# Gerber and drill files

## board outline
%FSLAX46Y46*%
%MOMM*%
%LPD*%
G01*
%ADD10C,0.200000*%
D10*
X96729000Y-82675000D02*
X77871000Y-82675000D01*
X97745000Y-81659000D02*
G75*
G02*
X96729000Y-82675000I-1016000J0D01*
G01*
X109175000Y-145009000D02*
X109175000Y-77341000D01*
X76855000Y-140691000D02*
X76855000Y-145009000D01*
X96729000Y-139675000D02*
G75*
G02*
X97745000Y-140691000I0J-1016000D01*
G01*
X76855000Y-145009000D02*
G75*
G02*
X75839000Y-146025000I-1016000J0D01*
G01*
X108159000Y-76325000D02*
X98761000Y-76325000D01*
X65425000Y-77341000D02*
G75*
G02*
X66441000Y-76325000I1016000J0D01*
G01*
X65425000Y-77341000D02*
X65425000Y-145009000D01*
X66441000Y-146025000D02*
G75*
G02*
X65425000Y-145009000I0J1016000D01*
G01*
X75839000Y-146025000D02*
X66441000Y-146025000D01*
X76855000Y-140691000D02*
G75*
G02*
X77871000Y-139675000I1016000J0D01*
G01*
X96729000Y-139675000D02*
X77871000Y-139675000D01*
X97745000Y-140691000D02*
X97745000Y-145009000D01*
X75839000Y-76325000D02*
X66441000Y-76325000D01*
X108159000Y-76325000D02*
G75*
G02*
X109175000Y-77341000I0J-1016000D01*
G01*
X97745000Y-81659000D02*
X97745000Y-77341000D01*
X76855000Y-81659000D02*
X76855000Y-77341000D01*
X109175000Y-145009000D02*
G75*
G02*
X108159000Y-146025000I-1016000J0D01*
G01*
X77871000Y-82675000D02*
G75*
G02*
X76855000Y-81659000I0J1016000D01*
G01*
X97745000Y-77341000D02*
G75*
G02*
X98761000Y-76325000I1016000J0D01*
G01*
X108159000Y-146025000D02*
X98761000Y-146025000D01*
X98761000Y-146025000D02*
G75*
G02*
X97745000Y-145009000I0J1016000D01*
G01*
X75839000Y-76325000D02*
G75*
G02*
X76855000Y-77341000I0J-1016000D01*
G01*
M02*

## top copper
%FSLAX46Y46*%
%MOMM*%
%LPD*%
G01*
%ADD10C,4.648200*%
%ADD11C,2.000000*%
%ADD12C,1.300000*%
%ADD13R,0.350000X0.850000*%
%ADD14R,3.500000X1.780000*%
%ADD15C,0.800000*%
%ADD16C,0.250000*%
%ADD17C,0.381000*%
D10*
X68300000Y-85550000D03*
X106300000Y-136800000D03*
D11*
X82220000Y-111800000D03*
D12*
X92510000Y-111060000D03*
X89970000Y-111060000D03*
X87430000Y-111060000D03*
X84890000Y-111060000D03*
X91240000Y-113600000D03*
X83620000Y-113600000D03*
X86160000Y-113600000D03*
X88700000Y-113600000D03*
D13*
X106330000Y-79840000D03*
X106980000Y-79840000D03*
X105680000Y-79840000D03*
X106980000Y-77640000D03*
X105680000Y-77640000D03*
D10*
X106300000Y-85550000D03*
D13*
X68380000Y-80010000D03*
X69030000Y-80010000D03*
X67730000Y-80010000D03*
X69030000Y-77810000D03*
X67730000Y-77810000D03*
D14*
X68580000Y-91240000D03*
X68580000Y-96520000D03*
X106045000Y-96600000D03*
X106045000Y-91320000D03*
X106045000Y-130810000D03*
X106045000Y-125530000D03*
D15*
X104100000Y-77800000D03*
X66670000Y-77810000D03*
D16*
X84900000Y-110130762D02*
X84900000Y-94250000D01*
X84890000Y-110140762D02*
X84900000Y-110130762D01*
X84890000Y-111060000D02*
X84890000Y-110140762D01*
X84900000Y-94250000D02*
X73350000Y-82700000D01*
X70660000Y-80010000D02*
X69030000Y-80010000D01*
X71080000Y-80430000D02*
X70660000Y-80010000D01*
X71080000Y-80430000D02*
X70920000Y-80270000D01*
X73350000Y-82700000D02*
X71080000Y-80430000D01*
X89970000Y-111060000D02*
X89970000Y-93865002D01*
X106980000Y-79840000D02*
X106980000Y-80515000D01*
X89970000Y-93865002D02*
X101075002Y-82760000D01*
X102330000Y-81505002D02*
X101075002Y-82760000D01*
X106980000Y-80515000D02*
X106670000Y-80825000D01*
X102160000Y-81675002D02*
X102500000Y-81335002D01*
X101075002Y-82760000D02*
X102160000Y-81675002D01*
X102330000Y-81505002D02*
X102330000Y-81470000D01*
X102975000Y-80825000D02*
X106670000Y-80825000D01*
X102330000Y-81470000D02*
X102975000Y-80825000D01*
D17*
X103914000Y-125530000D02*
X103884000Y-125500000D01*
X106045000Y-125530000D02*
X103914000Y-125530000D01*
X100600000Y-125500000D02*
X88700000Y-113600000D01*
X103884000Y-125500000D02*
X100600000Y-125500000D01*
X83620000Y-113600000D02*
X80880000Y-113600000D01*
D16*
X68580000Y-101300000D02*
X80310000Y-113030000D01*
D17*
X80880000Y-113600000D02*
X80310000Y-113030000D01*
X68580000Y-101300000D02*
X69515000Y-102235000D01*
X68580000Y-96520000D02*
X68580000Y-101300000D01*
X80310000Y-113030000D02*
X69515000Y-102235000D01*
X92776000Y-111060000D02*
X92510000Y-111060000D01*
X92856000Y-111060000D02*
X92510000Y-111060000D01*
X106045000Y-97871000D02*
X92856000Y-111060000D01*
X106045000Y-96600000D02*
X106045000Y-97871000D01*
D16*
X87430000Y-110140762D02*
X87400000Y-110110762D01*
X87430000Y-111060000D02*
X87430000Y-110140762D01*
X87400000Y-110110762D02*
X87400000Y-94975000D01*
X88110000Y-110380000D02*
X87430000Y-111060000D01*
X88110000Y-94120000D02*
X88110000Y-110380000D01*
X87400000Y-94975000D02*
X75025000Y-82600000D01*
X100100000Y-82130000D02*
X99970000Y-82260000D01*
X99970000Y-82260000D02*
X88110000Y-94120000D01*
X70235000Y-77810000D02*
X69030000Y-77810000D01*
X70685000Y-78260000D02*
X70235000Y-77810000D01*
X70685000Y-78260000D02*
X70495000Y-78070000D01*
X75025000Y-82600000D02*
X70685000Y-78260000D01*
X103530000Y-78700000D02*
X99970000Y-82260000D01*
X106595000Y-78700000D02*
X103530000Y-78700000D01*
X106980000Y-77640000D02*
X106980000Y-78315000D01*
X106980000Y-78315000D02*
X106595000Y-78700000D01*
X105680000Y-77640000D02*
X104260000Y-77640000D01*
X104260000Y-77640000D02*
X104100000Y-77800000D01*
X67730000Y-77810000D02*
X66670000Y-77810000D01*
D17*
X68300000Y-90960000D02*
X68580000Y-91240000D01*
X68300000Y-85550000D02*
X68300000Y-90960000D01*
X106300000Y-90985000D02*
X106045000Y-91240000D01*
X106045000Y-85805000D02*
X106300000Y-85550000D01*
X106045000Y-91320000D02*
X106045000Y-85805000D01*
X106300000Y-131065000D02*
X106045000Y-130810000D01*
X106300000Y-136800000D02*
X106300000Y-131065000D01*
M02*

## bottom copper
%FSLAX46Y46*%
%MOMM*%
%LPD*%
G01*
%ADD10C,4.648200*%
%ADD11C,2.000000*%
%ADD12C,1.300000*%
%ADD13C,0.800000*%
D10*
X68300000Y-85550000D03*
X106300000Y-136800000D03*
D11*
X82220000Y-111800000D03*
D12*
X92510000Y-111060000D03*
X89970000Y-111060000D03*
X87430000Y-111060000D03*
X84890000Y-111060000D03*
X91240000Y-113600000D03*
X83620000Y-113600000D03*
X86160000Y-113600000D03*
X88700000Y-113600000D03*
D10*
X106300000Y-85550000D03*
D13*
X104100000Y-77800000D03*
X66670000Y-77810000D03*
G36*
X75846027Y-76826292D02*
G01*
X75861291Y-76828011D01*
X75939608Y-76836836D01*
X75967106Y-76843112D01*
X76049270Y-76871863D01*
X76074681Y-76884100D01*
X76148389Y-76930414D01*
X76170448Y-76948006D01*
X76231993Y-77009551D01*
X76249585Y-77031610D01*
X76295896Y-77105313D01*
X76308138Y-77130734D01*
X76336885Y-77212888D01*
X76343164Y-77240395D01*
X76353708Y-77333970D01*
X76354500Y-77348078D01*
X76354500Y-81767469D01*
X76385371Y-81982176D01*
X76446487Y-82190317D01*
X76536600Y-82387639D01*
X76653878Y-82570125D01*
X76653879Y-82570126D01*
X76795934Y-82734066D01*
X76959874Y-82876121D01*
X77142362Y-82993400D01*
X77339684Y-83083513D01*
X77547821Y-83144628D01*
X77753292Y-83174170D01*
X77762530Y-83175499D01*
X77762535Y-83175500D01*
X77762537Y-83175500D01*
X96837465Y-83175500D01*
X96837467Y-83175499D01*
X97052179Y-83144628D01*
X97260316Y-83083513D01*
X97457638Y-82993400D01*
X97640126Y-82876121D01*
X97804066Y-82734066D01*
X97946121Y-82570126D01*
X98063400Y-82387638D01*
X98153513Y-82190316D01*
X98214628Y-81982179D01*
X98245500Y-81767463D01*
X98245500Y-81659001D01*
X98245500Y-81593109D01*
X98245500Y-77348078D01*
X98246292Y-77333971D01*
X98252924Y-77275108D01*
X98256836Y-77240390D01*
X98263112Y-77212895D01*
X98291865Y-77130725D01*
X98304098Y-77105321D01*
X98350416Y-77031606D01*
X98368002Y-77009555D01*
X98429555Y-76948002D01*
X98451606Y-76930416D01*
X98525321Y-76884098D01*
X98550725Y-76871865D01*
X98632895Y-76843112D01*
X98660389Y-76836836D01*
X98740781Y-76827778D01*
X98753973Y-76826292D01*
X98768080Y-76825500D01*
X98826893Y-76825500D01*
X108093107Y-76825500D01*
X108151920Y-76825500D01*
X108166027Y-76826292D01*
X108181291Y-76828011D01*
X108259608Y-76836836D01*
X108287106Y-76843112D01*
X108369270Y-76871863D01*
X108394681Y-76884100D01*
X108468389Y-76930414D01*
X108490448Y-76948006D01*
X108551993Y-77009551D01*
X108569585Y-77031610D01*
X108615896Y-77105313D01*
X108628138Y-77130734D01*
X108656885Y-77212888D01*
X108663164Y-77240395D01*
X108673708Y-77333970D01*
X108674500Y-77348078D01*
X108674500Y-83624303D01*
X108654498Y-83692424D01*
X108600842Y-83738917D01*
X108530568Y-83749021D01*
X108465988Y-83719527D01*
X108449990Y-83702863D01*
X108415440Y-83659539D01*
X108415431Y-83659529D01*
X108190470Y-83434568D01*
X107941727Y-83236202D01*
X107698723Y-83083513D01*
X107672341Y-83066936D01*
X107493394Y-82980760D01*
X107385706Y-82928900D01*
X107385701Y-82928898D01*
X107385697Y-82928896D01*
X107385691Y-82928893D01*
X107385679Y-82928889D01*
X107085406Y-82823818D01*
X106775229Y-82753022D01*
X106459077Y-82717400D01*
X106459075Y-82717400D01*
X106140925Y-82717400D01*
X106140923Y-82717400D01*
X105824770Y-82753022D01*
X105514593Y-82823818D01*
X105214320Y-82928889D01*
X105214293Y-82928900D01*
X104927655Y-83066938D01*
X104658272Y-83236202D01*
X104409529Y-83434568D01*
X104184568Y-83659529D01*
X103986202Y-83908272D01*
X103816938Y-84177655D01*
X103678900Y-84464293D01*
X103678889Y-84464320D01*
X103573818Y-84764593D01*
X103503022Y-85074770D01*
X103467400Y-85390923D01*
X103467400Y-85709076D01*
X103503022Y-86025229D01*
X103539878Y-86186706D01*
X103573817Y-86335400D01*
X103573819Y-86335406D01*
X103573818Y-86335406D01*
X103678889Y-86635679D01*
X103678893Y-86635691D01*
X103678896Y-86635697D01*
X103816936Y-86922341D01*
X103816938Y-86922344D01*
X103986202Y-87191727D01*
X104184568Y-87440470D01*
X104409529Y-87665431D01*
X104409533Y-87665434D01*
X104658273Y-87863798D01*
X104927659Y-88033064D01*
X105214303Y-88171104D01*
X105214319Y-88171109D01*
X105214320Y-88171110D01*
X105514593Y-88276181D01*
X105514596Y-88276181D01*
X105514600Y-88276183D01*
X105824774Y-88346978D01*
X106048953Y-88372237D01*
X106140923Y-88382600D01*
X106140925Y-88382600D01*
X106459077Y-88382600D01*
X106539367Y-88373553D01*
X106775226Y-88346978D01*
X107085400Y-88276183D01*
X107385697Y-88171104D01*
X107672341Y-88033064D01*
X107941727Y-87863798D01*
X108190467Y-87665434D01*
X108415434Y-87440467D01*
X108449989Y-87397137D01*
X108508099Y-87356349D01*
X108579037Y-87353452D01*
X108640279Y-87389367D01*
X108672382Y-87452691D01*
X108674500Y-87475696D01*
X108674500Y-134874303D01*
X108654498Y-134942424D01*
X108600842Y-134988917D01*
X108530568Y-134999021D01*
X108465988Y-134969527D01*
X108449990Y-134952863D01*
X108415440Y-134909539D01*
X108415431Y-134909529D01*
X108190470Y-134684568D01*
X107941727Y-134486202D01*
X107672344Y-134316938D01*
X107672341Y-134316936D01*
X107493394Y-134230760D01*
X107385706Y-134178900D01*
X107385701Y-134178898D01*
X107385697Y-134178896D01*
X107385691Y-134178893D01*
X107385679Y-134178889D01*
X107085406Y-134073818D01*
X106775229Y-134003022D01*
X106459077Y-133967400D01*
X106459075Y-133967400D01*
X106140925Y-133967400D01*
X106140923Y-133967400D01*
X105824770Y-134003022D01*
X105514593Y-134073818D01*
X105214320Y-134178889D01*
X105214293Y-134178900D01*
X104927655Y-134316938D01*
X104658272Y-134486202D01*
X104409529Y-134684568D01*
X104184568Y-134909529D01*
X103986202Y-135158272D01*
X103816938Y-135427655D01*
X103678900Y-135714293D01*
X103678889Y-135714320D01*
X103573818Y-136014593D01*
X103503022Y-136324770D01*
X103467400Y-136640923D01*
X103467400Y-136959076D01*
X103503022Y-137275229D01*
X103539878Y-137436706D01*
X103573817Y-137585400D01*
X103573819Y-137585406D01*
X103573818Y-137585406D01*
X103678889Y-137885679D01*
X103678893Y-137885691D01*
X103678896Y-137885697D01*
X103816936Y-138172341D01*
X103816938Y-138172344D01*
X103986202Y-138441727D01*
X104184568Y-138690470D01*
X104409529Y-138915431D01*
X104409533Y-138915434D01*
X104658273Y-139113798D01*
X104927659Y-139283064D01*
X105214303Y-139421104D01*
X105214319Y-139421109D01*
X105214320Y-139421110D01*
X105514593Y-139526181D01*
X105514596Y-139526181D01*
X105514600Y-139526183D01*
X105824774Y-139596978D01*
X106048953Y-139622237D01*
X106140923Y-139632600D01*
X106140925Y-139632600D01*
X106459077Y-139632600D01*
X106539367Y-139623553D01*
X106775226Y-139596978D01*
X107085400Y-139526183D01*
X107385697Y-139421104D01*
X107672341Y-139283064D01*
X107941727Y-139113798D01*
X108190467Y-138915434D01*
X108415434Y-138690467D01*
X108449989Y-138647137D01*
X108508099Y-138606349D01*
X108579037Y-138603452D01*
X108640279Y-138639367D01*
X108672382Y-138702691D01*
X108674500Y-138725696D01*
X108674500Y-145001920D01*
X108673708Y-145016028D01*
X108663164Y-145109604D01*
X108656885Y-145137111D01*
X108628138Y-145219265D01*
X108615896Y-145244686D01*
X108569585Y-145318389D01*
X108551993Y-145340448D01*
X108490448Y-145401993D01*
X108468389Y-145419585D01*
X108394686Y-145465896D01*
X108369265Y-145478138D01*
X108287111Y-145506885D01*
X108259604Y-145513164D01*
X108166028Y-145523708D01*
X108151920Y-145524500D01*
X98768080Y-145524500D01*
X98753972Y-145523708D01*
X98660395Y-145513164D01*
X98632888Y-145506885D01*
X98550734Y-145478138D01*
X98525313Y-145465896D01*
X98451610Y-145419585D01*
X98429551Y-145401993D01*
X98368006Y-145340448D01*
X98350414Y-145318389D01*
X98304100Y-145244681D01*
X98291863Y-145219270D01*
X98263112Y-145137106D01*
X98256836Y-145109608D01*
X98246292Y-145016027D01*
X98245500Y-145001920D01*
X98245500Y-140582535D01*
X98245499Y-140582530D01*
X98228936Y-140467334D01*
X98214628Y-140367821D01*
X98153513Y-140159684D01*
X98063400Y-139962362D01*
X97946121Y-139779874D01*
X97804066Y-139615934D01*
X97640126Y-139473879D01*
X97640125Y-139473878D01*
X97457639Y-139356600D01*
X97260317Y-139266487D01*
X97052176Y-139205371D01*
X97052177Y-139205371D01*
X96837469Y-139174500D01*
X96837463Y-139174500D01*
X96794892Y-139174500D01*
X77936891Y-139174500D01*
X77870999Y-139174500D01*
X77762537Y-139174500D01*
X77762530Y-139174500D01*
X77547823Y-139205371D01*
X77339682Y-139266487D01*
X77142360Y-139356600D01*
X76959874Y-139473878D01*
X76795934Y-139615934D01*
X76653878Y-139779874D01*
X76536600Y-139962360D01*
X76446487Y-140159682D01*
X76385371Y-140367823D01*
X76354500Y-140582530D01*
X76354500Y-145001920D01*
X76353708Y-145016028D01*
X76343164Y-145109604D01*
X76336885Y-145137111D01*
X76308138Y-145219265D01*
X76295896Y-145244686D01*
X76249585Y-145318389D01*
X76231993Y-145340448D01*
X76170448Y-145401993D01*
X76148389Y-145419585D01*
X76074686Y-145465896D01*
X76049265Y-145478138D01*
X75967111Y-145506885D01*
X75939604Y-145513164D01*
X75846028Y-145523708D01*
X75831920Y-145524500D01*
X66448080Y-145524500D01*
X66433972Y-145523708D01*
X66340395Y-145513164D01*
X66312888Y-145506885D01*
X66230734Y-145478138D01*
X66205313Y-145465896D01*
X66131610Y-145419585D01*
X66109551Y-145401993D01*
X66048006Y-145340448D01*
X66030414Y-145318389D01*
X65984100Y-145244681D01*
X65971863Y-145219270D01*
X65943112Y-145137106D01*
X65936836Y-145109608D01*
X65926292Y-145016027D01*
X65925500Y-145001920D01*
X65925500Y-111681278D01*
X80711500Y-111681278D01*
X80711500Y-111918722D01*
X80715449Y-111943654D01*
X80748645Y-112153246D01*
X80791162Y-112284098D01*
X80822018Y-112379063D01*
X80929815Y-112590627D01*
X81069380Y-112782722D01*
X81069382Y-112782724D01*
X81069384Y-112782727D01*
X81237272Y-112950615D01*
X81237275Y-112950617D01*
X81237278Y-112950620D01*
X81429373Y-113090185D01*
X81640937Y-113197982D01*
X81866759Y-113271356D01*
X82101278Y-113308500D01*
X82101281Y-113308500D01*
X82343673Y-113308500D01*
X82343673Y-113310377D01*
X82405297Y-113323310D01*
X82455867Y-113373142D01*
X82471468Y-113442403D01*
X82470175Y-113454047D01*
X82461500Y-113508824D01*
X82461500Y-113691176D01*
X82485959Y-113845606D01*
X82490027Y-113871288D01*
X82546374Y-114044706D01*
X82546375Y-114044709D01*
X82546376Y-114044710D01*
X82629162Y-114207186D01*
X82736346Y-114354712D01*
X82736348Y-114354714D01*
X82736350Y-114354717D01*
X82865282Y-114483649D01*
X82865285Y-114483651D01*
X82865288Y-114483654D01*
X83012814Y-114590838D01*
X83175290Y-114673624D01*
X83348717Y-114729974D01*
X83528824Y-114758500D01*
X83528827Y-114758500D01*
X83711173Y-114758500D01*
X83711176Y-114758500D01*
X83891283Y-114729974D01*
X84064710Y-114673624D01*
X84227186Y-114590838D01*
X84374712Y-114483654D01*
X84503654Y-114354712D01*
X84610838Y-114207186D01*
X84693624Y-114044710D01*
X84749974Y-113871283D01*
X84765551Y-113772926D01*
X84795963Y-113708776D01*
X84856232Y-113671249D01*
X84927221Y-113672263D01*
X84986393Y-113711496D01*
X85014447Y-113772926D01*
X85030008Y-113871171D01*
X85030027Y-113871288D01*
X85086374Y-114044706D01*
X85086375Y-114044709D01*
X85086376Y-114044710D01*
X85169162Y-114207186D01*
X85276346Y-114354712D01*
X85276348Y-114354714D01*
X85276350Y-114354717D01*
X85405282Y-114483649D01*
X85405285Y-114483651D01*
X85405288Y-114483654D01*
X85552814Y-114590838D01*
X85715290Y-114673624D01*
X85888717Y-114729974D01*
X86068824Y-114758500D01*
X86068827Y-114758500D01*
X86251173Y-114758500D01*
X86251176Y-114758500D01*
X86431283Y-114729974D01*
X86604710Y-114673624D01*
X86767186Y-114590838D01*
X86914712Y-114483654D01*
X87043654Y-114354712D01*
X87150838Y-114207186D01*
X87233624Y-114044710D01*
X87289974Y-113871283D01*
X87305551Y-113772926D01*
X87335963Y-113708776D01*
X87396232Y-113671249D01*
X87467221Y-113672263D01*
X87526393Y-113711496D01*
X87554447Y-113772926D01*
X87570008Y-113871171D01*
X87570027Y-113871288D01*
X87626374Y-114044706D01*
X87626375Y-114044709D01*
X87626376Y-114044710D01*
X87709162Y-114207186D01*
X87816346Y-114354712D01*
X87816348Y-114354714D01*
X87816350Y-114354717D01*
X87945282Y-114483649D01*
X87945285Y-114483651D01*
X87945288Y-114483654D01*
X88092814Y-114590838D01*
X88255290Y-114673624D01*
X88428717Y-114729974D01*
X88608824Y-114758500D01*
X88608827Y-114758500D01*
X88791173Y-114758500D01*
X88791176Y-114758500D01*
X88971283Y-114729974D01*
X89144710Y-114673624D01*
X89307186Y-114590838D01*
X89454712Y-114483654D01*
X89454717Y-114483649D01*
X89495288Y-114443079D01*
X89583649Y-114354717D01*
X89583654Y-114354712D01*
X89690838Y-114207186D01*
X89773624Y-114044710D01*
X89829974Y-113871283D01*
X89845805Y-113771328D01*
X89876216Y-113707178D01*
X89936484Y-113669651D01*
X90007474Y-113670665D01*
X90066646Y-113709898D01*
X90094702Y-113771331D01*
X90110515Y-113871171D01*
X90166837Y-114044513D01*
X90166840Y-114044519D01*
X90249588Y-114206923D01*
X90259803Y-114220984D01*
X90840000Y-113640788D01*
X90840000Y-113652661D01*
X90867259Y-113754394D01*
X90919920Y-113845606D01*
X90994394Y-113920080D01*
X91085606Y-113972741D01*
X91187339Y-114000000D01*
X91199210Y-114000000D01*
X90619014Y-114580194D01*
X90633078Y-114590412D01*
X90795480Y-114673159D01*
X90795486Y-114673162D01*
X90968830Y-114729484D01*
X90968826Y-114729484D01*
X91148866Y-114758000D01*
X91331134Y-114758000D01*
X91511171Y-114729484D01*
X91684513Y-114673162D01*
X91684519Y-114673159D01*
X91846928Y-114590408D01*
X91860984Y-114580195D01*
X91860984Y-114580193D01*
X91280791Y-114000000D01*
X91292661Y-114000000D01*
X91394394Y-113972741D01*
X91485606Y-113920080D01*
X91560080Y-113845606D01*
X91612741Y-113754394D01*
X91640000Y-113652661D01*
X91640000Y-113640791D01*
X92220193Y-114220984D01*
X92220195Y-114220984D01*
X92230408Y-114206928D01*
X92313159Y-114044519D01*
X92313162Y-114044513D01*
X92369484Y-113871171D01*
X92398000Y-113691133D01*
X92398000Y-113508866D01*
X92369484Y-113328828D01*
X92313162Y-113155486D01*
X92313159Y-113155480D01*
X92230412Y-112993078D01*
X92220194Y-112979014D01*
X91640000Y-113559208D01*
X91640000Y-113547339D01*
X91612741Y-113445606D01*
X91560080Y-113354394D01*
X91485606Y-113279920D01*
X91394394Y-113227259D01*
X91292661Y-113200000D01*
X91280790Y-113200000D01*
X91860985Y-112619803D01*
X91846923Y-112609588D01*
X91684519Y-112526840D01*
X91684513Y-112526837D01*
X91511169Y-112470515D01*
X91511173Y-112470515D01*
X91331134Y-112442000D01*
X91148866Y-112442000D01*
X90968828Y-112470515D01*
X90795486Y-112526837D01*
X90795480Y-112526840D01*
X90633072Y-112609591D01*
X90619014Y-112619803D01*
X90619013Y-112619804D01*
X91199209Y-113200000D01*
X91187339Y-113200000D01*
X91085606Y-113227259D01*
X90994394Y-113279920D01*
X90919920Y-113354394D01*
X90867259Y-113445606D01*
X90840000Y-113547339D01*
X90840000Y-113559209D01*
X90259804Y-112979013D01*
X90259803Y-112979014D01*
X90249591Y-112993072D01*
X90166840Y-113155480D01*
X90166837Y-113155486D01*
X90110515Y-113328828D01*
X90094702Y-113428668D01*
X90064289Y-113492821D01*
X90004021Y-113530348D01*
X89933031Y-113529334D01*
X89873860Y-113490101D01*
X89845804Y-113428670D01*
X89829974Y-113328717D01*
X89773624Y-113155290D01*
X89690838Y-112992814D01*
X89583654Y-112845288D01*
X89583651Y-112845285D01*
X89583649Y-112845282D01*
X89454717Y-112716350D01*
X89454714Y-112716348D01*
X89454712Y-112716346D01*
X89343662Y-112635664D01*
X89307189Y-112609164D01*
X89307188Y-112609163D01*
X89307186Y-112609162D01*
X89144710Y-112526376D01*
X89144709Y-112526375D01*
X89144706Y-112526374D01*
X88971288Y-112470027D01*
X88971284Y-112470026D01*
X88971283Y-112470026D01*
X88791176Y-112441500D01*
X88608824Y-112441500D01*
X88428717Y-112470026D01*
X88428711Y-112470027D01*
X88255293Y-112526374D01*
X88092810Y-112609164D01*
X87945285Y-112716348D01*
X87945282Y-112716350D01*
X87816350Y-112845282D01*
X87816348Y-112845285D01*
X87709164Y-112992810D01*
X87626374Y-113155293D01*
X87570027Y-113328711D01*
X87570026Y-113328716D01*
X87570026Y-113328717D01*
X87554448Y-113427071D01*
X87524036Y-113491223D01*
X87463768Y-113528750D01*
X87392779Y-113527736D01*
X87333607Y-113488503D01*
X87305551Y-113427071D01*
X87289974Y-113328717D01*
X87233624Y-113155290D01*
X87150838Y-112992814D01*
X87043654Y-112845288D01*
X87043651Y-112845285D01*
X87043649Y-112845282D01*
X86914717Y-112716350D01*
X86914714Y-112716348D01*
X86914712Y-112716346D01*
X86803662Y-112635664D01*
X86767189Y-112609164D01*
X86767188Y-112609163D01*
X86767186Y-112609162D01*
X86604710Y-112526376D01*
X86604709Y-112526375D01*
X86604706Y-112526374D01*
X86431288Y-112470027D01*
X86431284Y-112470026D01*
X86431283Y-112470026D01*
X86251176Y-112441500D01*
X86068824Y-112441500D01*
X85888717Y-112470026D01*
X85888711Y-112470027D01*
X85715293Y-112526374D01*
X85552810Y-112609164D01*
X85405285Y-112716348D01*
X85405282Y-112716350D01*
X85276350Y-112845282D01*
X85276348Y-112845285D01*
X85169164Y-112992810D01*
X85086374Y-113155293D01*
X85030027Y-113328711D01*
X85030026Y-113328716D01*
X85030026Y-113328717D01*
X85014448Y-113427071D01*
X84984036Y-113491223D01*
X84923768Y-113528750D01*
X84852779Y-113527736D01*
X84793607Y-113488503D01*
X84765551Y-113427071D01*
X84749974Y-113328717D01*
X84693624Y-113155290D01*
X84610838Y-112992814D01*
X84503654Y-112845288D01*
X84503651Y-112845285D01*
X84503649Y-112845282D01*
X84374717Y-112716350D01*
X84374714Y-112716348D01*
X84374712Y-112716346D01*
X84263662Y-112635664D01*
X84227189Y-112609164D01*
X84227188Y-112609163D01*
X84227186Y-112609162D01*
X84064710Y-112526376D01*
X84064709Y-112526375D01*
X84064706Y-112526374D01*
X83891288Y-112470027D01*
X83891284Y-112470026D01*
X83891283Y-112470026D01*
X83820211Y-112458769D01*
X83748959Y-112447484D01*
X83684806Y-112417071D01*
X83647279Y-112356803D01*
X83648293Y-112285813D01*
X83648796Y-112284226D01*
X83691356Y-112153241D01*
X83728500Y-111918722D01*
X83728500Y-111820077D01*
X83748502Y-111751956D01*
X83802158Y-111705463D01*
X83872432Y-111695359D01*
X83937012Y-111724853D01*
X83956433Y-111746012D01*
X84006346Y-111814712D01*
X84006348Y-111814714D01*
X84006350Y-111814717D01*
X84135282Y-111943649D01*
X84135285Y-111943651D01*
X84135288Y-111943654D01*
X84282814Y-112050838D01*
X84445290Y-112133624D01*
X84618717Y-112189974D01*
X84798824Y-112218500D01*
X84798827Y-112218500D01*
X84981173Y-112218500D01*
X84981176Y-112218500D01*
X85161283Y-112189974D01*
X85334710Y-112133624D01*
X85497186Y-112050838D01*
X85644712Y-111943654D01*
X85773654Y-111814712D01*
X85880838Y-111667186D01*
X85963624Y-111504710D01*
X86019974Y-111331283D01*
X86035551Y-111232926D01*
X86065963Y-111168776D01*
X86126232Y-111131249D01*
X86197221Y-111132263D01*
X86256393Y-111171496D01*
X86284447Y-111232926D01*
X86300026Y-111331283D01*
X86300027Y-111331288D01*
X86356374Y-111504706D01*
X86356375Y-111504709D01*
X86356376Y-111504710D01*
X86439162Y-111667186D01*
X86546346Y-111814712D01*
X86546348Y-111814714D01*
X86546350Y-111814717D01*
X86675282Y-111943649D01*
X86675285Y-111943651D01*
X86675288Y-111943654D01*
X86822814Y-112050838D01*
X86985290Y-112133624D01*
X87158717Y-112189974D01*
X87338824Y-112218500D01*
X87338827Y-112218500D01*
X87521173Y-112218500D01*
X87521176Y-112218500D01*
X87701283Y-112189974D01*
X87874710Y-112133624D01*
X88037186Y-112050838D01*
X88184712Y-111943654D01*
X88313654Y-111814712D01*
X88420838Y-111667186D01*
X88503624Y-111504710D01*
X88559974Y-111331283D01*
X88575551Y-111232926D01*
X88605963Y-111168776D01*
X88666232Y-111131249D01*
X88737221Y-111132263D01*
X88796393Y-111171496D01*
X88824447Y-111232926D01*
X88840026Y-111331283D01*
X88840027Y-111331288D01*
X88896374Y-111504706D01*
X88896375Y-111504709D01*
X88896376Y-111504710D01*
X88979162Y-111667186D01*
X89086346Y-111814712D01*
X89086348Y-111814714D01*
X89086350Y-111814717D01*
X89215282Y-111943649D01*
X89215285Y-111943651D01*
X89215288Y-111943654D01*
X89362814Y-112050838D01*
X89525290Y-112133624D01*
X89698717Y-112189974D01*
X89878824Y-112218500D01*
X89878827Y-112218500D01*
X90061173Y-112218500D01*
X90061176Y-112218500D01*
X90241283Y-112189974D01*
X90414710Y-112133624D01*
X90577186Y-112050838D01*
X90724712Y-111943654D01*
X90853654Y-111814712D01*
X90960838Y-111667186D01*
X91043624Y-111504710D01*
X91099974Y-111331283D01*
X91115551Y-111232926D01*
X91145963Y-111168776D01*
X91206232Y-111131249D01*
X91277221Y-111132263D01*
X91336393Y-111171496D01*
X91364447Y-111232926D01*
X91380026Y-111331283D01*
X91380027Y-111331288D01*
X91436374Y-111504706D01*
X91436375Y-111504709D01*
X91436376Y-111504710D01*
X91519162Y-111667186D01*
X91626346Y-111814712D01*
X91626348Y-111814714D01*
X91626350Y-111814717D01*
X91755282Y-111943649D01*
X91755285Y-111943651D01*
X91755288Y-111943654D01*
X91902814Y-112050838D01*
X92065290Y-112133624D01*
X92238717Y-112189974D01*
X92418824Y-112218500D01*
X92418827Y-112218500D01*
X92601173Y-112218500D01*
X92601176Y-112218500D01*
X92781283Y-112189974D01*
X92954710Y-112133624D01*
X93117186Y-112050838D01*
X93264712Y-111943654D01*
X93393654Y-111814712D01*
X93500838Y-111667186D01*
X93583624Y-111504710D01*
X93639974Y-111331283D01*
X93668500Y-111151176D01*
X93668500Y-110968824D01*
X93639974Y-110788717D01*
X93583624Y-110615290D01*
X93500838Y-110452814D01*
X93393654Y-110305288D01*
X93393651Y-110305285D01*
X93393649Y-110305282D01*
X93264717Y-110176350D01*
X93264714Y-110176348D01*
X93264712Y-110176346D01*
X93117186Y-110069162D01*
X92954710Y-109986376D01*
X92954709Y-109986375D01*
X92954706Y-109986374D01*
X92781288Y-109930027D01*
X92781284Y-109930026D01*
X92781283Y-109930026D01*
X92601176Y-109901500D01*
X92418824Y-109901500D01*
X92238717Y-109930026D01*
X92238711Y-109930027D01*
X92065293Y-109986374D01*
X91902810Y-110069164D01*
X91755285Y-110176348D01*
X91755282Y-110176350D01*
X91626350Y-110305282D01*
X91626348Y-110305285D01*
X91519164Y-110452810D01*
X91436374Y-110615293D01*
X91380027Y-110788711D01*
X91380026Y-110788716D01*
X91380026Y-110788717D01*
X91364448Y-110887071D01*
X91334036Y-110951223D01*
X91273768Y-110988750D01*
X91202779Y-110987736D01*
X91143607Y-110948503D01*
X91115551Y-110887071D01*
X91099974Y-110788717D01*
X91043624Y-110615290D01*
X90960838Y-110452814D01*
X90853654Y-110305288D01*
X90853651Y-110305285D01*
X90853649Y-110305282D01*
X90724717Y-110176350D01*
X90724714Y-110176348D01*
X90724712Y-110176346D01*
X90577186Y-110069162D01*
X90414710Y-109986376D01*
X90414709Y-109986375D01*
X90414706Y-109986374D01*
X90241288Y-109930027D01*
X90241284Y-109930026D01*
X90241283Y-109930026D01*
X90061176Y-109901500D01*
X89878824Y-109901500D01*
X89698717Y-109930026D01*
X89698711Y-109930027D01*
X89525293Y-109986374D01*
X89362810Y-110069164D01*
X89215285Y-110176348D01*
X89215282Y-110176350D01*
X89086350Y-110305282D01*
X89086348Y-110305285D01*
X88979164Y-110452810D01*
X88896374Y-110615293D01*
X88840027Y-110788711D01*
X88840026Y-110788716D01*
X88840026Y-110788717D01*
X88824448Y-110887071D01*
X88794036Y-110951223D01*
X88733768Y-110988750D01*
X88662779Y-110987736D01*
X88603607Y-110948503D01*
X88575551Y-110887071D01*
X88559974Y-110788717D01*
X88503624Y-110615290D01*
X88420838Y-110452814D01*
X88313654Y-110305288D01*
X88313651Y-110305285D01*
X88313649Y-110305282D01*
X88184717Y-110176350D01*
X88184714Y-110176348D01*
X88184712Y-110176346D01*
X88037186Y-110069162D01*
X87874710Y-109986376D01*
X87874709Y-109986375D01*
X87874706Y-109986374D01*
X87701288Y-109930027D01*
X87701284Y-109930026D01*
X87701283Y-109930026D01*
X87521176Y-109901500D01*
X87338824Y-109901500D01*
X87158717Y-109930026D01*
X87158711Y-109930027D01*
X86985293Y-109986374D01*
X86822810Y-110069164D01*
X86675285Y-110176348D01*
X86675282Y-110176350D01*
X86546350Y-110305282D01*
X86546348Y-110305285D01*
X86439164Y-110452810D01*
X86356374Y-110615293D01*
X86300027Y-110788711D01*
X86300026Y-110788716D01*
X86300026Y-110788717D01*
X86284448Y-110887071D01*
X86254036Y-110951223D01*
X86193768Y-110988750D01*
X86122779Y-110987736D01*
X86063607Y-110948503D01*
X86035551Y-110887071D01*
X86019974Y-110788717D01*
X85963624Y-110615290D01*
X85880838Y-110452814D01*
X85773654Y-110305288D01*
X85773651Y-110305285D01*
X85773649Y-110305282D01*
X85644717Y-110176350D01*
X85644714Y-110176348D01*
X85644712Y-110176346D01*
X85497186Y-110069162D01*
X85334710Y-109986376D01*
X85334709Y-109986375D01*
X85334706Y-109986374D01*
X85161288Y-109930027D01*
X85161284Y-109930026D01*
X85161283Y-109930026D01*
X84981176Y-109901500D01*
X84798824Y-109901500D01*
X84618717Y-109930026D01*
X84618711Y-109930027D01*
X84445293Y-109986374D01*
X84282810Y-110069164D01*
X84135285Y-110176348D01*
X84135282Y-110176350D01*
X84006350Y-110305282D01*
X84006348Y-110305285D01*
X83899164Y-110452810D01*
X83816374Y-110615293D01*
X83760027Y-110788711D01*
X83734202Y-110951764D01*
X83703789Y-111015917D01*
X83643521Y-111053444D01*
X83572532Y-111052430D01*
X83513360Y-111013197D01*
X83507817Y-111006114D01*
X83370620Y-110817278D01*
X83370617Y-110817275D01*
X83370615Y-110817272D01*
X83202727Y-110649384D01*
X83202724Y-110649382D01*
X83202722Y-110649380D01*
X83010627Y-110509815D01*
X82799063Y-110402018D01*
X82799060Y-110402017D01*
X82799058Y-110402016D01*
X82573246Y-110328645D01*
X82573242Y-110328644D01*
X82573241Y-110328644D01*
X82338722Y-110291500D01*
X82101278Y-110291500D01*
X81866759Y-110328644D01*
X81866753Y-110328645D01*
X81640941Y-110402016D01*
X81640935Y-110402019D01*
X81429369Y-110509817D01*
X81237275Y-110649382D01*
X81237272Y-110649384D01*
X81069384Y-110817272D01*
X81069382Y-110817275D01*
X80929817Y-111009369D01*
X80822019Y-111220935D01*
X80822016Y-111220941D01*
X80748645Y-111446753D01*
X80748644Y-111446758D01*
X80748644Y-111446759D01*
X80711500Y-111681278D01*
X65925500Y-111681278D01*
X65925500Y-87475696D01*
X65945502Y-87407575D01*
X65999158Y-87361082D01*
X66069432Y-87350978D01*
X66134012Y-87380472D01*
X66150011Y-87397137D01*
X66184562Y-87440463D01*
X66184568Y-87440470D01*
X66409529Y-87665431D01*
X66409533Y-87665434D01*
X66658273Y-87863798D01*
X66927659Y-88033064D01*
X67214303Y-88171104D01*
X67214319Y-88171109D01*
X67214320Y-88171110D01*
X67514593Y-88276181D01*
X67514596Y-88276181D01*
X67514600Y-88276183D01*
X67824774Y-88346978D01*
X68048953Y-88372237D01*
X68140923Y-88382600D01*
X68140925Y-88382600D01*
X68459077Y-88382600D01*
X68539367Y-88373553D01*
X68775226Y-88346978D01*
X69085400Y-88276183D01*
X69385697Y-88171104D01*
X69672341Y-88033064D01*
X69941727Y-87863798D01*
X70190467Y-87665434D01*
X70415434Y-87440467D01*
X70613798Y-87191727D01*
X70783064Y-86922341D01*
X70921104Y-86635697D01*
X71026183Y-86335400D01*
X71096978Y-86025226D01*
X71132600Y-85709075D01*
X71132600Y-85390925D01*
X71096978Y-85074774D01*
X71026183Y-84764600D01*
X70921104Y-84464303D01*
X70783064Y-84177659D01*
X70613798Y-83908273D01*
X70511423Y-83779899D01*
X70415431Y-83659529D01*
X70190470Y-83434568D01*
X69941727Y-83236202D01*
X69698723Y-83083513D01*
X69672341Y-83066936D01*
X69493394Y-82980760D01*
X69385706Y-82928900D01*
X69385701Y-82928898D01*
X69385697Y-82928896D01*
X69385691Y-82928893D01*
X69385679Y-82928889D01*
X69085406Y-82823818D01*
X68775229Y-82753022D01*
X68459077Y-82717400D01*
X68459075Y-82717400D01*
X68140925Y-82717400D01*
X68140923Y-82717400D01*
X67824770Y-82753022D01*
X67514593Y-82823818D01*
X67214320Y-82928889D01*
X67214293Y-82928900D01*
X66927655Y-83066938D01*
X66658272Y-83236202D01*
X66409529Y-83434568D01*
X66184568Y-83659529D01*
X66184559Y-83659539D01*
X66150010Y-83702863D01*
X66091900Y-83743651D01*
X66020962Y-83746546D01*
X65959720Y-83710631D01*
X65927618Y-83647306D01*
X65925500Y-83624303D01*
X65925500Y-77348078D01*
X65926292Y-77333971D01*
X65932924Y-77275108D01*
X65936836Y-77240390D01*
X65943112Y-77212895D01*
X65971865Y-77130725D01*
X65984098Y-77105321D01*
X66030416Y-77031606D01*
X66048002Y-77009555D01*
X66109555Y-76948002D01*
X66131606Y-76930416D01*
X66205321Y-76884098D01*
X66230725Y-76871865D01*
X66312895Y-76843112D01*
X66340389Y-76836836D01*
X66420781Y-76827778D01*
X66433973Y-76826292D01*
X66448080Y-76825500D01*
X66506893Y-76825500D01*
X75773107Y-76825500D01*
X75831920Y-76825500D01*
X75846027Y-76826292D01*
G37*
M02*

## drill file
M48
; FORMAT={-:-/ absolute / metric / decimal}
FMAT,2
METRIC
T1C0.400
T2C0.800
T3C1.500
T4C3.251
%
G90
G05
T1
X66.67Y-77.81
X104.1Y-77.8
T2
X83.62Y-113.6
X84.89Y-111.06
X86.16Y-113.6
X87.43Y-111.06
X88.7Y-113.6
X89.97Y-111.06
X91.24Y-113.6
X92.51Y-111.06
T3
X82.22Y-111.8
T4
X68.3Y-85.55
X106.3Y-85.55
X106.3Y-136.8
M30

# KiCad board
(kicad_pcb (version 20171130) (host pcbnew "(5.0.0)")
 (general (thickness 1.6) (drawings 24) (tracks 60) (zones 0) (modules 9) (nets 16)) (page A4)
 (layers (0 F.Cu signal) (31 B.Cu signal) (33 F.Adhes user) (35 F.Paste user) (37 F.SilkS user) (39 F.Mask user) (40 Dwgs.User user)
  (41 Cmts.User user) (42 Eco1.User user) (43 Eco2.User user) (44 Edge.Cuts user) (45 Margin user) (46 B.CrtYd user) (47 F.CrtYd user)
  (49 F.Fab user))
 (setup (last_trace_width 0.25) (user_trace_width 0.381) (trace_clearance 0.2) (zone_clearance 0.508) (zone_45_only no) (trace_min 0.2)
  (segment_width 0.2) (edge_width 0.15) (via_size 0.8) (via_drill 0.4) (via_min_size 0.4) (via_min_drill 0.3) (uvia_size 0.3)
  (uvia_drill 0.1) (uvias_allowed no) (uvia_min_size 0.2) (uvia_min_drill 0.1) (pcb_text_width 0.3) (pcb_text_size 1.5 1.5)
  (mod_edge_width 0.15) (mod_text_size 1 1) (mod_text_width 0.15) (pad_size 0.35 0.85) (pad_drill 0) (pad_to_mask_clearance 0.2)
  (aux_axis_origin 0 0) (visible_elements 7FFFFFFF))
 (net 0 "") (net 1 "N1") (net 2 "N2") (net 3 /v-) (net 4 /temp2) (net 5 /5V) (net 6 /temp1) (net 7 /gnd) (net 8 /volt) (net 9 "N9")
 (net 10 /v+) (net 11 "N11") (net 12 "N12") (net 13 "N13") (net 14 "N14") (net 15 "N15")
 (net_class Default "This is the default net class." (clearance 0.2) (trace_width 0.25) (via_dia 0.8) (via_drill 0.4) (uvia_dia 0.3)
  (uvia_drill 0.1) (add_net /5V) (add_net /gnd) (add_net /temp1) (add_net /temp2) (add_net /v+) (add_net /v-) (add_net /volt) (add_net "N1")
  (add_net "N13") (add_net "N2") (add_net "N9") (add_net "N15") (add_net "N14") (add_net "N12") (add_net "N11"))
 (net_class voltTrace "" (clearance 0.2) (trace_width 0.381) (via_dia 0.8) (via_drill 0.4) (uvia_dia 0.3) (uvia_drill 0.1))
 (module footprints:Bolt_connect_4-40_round (layer F.Cu) (at 68.3 85.55)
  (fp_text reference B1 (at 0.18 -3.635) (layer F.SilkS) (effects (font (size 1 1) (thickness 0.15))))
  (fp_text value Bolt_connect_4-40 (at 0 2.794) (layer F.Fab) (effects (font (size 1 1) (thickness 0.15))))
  (pad 1 thru_hole circle (at 0 0) (size 4.6482 4.6482) (drill 3.2512) (layers *.Cu *.Mask) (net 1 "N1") (clearance 0.508)))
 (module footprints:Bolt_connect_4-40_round (layer F.Cu) (at 106.3 136.8)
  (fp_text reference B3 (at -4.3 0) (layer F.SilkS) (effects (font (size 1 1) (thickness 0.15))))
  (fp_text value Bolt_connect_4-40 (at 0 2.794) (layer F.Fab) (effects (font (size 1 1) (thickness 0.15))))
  (pad 1 thru_hole circle (at 0 0) (size 4.6482 4.6482) (drill 3.2512) (layers *.Cu *.Mask) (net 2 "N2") (clearance 0.508)))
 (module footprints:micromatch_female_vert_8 (layer F.Cu) (at 88.7 113.6 90)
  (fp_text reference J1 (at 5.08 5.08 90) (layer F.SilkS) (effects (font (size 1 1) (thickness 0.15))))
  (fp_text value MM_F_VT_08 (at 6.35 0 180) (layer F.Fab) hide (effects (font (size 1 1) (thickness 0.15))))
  (pad 9 thru_hole circle (at 1.8 -6.48 90) (size 2 2) (drill 1.5) (layers *.Cu *.Mask))
  (pad 8 thru_hole circle (at 2.54 3.81 90) (size 1.3 1.3) (drill 0.8) (layers *.Cu *.Mask) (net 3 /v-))
  (pad 6 thru_hole circle (at 2.54 1.27 90) (size 1.3 1.3) (drill 0.8) (layers *.Cu *.Mask) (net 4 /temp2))
  (pad 4 thru_hole circle (at 2.54 -1.27 90) (size 1.3 1.3) (drill 0.8) (layers *.Cu *.Mask) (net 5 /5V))
  (pad 2 thru_hole circle (at 2.54 -3.81 90) (size 1.3 1.3) (drill 0.8) (layers *.Cu *.Mask) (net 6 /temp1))
  (pad 7 thru_hole circle (at 0 2.54 90) (size 1.3 1.3) (drill 0.8) (layers *.Cu *.Mask) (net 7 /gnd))
  (pad 1 thru_hole circle (at 0 -5.08 90) (size 1.3 1.3) (drill 0.8) (layers *.Cu *.Mask) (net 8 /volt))
  (pad 3 thru_hole circle (at 0 -2.54 90) (size 1.3 1.3) (drill 0.8) (layers *.Cu *.Mask) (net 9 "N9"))
  (pad 5 thru_hole circle (at 0 0 90) (size 1.3 1.3) (drill 0.8) (layers *.Cu *.Mask) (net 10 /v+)))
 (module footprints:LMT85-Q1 (layer F.Cu) (at 105.68 79.84)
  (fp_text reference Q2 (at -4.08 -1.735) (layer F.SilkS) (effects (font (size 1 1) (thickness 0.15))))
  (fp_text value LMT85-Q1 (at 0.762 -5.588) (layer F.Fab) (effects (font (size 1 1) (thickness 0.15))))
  (pad 3 smd rect (at 0.65 0) (size 0.35 0.85) (layers F.Cu F.Paste F.Mask) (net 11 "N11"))
  (pad 4 smd rect (at 1.3 0) (size 0.35 0.85) (layers F.Cu F.Paste F.Mask) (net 4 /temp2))
  (pad 2 smd rect (at 0 0) (size 0.35 0.85) (layers F.Cu F.Paste F.Mask) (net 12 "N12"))
  (pad 5 smd rect (at 1.3 -2.2) (size 0.35 0.85) (layers F.Cu F.Paste F.Mask) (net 5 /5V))
  (pad 1 smd rect (at 0 -2.2) (size 0.35 0.85) (layers F.Cu F.Paste F.Mask) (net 7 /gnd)))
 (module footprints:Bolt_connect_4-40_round (layer F.Cu) (at 106.3 85.55)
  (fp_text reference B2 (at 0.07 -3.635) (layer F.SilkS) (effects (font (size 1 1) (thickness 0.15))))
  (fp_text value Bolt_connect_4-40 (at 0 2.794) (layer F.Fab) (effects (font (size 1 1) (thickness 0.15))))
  (pad 1 thru_hole circle (at 0 0) (size 4.6482 4.6482) (drill 3.2512) (layers *.Cu *.Mask) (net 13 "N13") (clearance 0.508)))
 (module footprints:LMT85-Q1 (layer F.Cu) (at 67.73 80.01)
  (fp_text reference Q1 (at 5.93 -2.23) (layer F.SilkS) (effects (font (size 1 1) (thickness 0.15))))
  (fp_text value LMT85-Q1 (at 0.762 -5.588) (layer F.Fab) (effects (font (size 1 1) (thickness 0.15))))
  (pad 3 smd rect (at 0.65 0) (size 0.35 0.85) (layers F.Cu F.Paste F.Mask) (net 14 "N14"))
  (pad 4 smd rect (at 1.3 0) (size 0.35 0.85) (layers F.Cu F.Paste F.Mask) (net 6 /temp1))
  (pad 2 smd rect (at 0 0) (size 0.35 0.85) (layers F.Cu F.Paste F.Mask) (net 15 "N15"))
  (pad 5 smd rect (at 1.3 -2.2) (size 0.35 0.85) (layers F.Cu F.Paste F.Mask) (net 5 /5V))
  (pad 1 smd rect (at 0 -2.2) (size 0.35 0.85) (layers F.Cu F.Paste F.Mask) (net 7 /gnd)))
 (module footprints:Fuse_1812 (layer F.Cu) (at 68.58 96.52 90)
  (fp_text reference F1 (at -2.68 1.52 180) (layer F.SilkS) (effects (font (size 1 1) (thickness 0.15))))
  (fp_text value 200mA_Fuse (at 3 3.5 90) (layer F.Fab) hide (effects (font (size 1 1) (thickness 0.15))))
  (pad 2 smd rect (at 5.28 0 90) (size 1.78 3.5) (layers F.Cu F.Paste F.Mask) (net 1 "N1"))
  (pad 1 smd rect (at 0 0 90) (size 1.78 3.5) (layers F.Cu F.Paste F.Mask) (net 8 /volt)))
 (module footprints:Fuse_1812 (layer F.Cu) (at 106.045 96.6 90)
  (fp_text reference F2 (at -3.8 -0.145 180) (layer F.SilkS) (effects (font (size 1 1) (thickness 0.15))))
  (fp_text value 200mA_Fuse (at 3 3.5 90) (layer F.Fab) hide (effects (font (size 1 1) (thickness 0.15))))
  (pad 1 smd rect (at 0 0 90) (size 1.78 3.5) (layers F.Cu F.Paste F.Mask) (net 3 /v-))
  (pad 2 smd rect (at 5.28 0 90) (size 1.78 3.5) (layers F.Cu F.Paste F.Mask) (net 13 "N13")))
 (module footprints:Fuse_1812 (layer F.Cu) (at 106.045 125.53 270)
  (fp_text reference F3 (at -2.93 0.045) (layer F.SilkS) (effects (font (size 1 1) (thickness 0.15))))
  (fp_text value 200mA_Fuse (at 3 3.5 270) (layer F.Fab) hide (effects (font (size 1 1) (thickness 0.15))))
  (pad 2 smd rect (at 5.28 0 270) (size 1.78 3.5) (layers F.Cu F.Paste F.Mask) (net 2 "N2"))
  (pad 1 smd rect (at 0 0 270) (size 1.78 3.5) (layers F.Cu F.Paste F.Mask) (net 10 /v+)))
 (gr_line (start 96.729 82.675) (end 77.871 82.675) (layer Edge.Cuts) (width 0.2))
 (gr_arc (start 96.729 81.659) (end 96.729 82.675) (angle -90) (layer Edge.Cuts) (width 0.2))
 (gr_line (start 109.175 145.009) (end 109.175 77.341) (layer Edge.Cuts) (width 0.2))
 (gr_line (start 76.855 140.691) (end 76.855 145.009) (layer Edge.Cuts) (width 0.2))
 (gr_arc (start 96.729 140.691) (end 97.745 140.691) (angle -90) (layer Edge.Cuts) (width 0.2))
 (gr_arc (start 75.839 145.009) (end 75.839 146.025) (angle -90) (layer Edge.Cuts) (width 0.2))
 (gr_line (start 108.159 76.325) (end 98.761 76.325) (layer Edge.Cuts) (width 0.2))
 (gr_arc (start 66.441 77.341) (end 66.441 76.325) (angle -90) (layer Edge.Cuts) (width 0.2))
 (gr_line (start 65.425 77.341) (end 65.425 145.009) (layer Edge.Cuts) (width 0.2))
 (gr_arc (start 66.441 145.009) (end 65.425 145.009) (angle -90) (layer Edge.Cuts) (width 0.2))
 (gr_line (start 75.839 146.025) (end 66.441 146.025) (layer Edge.Cuts) (width 0.2))
 (gr_arc (start 77.871 140.691) (end 77.871 139.675) (angle -90) (layer Edge.Cuts) (width 0.2))
 (gr_line (start 96.729 139.675) (end 77.871 139.675) (layer Edge.Cuts) (width 0.2))
 (gr_line (start 97.745 140.691) (end 97.745 145.009) (layer Edge.Cuts) (width 0.2))
 (gr_line (start 75.839 76.325) (end 66.441 76.325) (layer Edge.Cuts) (width 0.2))
 (gr_arc (start 108.159 77.341) (end 109.175 77.341) (angle -90) (layer Edge.Cuts) (width 0.2))
 (gr_line (start 97.745 81.659) (end 97.745 77.341) (layer Edge.Cuts) (width 0.2))
 (gr_line (start 76.855 81.659) (end 76.855 77.341) (layer Edge.Cuts) (width 0.2))
 (gr_arc (start 108.159 145.009) (end 108.159 146.025) (angle -90) (layer Edge.Cuts) (width 0.2))
 (gr_arc (start 77.871 81.659) (end 76.855 81.659) (angle -90) (layer Edge.Cuts) (width 0.2))
 (gr_arc (start 98.761 77.341) (end 98.761 76.325) (angle -90) (layer Edge.Cuts) (width 0.2))
 (gr_line (start 108.159 146.025) (end 98.761 146.025) (layer Edge.Cuts) (width 0.2))
 (gr_arc (start 98.761 145.009) (end 97.745 145.009) (angle -90) (layer Edge.Cuts) (width 0.2))
 (gr_arc (start 75.839 77.341) (end 76.855 77.341) (angle -90) (layer Edge.Cuts) (width 0.2))
 (segment (start 84.9 110.130762) (end 84.9 94.25) (width 0.25) (layer F.Cu) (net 6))
 (segment (start 84.89 110.140762) (end 84.9 110.130762) (width 0.25) (layer F.Cu) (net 6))
 (segment (start 84.89 111.06) (end 84.89 110.140762) (width 0.25) (layer F.Cu) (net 6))
 (segment (start 84.9 94.25) (end 73.35 82.7) (width 0.25) (layer F.Cu) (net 6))
 (segment (start 70.66 80.01) (end 69.03 80.01) (width 0.25) (layer F.Cu) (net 6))
 (segment (start 71.08 80.43) (end 70.66 80.01) (width 0.25) (layer F.Cu) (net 6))
 (segment (start 71.08 80.43) (end 70.92 80.27) (width 0.25) (layer F.Cu) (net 6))
 (segment (start 73.35 82.7) (end 71.08 80.43) (width 0.25) (layer F.Cu) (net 6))
 (segment (start 89.97 111.06) (end 89.97 93.865002) (width 0.25) (layer F.Cu) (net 4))
 (segment (start 106.98 79.84) (end 106.98 80.515) (width 0.25) (layer F.Cu) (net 4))
 (segment (start 89.97 93.865002) (end 101.075002 82.76) (width 0.25) (layer F.Cu) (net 4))
 (segment (start 102.33 81.505002) (end 101.075002 82.76) (width 0.25) (layer F.Cu) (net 4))
 (segment (start 106.98 80.515) (end 106.67 80.825) (width 0.25) (layer F.Cu) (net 4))
 (segment (start 102.16 81.675002) (end 102.5 81.335002) (width 0.25) (layer F.Cu) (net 4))
 (segment (start 101.075002 82.76) (end 102.16 81.675002) (width 0.25) (layer F.Cu) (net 4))
 (segment (start 102.33 81.505002) (end 102.33 81.47) (width 0.25) (layer F.Cu) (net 4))
 (segment (start 102.975 80.825) (end 106.67 80.825) (width 0.25) (layer F.Cu) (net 4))
 (segment (start 102.33 81.47) (end 102.975 80.825) (width 0.25) (layer F.Cu) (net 4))
 (segment (start 103.914 125.53) (end 103.884 125.5) (width 0.381) (layer F.Cu) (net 10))
 (segment (start 106.045 125.53) (end 103.914 125.53) (width 0.381) (layer F.Cu) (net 10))
 (segment (start 100.6 125.5) (end 88.7 113.6) (width 0.381) (layer F.Cu) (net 10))
 (segment (start 103.884 125.5) (end 100.6 125.5) (width 0.381) (layer F.Cu) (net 10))
 (segment (start 83.62 113.6) (end 80.88 113.6) (width 0.381) (layer F.Cu) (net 8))
 (segment (start 68.58 101.3) (end 80.31 113.03) (width 0.25) (layer F.Cu) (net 8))
 (segment (start 80.88 113.6) (end 80.31 113.03) (width 0.381) (layer F.Cu) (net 8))
 (segment (start 68.58 101.3) (end 69.515 102.235) (width 0.381) (layer F.Cu) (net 8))
 (segment (start 68.58 96.52) (end 68.58 101.3) (width 0.381) (layer F.Cu) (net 8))
 (segment (start 80.31 113.03) (end 69.515 102.235) (width 0.381) (layer F.Cu) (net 8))
 (segment (start 92.776 111.06) (end 92.51 111.06) (width 0.381) (layer F.Cu) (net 3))
 (segment (start 92.856 111.06) (end 92.51 111.06) (width 0.381) (layer F.Cu) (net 3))
 (segment (start 106.045 97.871) (end 92.856 111.06) (width 0.381) (layer F.Cu) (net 3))
 (segment (start 106.045 96.6) (end 106.045 97.871) (width 0.381) (layer F.Cu) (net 3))
 (segment (start 87.43 110.140762) (end 87.4 110.110762) (width 0.25) (layer F.Cu) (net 5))
 (segment (start 87.43 111.06) (end 87.43 110.140762) (width 0.25) (layer F.Cu) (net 5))
 (segment (start 87.4 110.110762) (end 87.4 94.975) (width 0.25) (layer F.Cu) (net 5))
 (segment (start 88.11 110.38) (end 87.43 111.06) (width 0.25) (layer F.Cu) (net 5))
 (segment (start 88.11 94.12) (end 88.11 110.38) (width 0.25) (layer F.Cu) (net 5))
 (segment (start 87.4 94.975) (end 75.025 82.6) (width 0.25) (layer F.Cu) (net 5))
 (segment (start 100.1 82.13) (end 99.97 82.26) (width 0.25) (layer F.Cu) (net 5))
 (segment (start 99.97 82.26) (end 88.11 94.12) (width 0.25) (layer F.Cu) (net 5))
 (segment (start 70.235 77.81) (end 69.03 77.81) (width 0.25) (layer F.Cu) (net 5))
 (segment (start 70.685 78.26) (end 70.235 77.81) (width 0.25) (layer F.Cu) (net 5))
 (segment (start 70.685 78.26) (end 70.495 78.07) (width 0.25) (layer F.Cu) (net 5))
 (segment (start 75.025 82.6) (end 70.685 78.26) (width 0.25) (layer F.Cu) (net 5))
 (segment (start 103.53 78.7) (end 99.97 82.26) (width 0.25) (layer F.Cu) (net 5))
 (segment (start 106.595 78.7) (end 103.53 78.7) (width 0.25) (layer F.Cu) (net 5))
 (segment (start 106.98 77.64) (end 106.98 78.315) (width 0.25) (layer F.Cu) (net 5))
 (segment (start 106.98 78.315) (end 106.595 78.7) (width 0.25) (layer F.Cu) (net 5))
 (via (at 104.1 77.8) (size 0.8) (drill 0.4) (layers F.Cu B.Cu) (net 7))
 (segment (start 105.68 77.64) (end 104.26 77.64) (width 0.25) (layer F.Cu) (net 7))
 (segment (start 104.26 77.64) (end 104.1 77.8) (width 0.25) (layer F.Cu) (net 7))
 (via (at 66.67 77.81) (size 0.8) (drill 0.4) (layers F.Cu B.Cu) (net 7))
 (segment (start 67.73 77.81) (end 66.67 77.81) (width 0.25) (layer F.Cu) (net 7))
 (segment (start 68.3 90.96) (end 68.58 91.24) (width 0.381) (layer F.Cu) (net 1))
 (segment (start 68.3 85.55) (end 68.3 90.96) (width 0.381) (layer F.Cu) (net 1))
 (segment (start 106.3 90.985) (end 106.045 91.24) (width 0.381) (layer F.Cu) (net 13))
 (segment (start 106.045 85.805) (end 106.3 85.55) (width 0.381) (layer F.Cu) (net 13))
 (segment (start 106.045 91.32) (end 106.045 85.805) (width 0.381) (layer F.Cu) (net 13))
 (segment (start 106.3 131.065) (end 106.045 130.81) (width 0.381) (layer F.Cu) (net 2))
 (segment (start 106.3 136.8) (end 106.3 131.065) (width 0.381) (layer F.Cu) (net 2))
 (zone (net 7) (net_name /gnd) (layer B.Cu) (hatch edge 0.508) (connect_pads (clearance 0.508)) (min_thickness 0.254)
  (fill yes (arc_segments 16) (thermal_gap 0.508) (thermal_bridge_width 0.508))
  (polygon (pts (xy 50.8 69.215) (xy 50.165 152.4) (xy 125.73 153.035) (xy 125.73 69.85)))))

